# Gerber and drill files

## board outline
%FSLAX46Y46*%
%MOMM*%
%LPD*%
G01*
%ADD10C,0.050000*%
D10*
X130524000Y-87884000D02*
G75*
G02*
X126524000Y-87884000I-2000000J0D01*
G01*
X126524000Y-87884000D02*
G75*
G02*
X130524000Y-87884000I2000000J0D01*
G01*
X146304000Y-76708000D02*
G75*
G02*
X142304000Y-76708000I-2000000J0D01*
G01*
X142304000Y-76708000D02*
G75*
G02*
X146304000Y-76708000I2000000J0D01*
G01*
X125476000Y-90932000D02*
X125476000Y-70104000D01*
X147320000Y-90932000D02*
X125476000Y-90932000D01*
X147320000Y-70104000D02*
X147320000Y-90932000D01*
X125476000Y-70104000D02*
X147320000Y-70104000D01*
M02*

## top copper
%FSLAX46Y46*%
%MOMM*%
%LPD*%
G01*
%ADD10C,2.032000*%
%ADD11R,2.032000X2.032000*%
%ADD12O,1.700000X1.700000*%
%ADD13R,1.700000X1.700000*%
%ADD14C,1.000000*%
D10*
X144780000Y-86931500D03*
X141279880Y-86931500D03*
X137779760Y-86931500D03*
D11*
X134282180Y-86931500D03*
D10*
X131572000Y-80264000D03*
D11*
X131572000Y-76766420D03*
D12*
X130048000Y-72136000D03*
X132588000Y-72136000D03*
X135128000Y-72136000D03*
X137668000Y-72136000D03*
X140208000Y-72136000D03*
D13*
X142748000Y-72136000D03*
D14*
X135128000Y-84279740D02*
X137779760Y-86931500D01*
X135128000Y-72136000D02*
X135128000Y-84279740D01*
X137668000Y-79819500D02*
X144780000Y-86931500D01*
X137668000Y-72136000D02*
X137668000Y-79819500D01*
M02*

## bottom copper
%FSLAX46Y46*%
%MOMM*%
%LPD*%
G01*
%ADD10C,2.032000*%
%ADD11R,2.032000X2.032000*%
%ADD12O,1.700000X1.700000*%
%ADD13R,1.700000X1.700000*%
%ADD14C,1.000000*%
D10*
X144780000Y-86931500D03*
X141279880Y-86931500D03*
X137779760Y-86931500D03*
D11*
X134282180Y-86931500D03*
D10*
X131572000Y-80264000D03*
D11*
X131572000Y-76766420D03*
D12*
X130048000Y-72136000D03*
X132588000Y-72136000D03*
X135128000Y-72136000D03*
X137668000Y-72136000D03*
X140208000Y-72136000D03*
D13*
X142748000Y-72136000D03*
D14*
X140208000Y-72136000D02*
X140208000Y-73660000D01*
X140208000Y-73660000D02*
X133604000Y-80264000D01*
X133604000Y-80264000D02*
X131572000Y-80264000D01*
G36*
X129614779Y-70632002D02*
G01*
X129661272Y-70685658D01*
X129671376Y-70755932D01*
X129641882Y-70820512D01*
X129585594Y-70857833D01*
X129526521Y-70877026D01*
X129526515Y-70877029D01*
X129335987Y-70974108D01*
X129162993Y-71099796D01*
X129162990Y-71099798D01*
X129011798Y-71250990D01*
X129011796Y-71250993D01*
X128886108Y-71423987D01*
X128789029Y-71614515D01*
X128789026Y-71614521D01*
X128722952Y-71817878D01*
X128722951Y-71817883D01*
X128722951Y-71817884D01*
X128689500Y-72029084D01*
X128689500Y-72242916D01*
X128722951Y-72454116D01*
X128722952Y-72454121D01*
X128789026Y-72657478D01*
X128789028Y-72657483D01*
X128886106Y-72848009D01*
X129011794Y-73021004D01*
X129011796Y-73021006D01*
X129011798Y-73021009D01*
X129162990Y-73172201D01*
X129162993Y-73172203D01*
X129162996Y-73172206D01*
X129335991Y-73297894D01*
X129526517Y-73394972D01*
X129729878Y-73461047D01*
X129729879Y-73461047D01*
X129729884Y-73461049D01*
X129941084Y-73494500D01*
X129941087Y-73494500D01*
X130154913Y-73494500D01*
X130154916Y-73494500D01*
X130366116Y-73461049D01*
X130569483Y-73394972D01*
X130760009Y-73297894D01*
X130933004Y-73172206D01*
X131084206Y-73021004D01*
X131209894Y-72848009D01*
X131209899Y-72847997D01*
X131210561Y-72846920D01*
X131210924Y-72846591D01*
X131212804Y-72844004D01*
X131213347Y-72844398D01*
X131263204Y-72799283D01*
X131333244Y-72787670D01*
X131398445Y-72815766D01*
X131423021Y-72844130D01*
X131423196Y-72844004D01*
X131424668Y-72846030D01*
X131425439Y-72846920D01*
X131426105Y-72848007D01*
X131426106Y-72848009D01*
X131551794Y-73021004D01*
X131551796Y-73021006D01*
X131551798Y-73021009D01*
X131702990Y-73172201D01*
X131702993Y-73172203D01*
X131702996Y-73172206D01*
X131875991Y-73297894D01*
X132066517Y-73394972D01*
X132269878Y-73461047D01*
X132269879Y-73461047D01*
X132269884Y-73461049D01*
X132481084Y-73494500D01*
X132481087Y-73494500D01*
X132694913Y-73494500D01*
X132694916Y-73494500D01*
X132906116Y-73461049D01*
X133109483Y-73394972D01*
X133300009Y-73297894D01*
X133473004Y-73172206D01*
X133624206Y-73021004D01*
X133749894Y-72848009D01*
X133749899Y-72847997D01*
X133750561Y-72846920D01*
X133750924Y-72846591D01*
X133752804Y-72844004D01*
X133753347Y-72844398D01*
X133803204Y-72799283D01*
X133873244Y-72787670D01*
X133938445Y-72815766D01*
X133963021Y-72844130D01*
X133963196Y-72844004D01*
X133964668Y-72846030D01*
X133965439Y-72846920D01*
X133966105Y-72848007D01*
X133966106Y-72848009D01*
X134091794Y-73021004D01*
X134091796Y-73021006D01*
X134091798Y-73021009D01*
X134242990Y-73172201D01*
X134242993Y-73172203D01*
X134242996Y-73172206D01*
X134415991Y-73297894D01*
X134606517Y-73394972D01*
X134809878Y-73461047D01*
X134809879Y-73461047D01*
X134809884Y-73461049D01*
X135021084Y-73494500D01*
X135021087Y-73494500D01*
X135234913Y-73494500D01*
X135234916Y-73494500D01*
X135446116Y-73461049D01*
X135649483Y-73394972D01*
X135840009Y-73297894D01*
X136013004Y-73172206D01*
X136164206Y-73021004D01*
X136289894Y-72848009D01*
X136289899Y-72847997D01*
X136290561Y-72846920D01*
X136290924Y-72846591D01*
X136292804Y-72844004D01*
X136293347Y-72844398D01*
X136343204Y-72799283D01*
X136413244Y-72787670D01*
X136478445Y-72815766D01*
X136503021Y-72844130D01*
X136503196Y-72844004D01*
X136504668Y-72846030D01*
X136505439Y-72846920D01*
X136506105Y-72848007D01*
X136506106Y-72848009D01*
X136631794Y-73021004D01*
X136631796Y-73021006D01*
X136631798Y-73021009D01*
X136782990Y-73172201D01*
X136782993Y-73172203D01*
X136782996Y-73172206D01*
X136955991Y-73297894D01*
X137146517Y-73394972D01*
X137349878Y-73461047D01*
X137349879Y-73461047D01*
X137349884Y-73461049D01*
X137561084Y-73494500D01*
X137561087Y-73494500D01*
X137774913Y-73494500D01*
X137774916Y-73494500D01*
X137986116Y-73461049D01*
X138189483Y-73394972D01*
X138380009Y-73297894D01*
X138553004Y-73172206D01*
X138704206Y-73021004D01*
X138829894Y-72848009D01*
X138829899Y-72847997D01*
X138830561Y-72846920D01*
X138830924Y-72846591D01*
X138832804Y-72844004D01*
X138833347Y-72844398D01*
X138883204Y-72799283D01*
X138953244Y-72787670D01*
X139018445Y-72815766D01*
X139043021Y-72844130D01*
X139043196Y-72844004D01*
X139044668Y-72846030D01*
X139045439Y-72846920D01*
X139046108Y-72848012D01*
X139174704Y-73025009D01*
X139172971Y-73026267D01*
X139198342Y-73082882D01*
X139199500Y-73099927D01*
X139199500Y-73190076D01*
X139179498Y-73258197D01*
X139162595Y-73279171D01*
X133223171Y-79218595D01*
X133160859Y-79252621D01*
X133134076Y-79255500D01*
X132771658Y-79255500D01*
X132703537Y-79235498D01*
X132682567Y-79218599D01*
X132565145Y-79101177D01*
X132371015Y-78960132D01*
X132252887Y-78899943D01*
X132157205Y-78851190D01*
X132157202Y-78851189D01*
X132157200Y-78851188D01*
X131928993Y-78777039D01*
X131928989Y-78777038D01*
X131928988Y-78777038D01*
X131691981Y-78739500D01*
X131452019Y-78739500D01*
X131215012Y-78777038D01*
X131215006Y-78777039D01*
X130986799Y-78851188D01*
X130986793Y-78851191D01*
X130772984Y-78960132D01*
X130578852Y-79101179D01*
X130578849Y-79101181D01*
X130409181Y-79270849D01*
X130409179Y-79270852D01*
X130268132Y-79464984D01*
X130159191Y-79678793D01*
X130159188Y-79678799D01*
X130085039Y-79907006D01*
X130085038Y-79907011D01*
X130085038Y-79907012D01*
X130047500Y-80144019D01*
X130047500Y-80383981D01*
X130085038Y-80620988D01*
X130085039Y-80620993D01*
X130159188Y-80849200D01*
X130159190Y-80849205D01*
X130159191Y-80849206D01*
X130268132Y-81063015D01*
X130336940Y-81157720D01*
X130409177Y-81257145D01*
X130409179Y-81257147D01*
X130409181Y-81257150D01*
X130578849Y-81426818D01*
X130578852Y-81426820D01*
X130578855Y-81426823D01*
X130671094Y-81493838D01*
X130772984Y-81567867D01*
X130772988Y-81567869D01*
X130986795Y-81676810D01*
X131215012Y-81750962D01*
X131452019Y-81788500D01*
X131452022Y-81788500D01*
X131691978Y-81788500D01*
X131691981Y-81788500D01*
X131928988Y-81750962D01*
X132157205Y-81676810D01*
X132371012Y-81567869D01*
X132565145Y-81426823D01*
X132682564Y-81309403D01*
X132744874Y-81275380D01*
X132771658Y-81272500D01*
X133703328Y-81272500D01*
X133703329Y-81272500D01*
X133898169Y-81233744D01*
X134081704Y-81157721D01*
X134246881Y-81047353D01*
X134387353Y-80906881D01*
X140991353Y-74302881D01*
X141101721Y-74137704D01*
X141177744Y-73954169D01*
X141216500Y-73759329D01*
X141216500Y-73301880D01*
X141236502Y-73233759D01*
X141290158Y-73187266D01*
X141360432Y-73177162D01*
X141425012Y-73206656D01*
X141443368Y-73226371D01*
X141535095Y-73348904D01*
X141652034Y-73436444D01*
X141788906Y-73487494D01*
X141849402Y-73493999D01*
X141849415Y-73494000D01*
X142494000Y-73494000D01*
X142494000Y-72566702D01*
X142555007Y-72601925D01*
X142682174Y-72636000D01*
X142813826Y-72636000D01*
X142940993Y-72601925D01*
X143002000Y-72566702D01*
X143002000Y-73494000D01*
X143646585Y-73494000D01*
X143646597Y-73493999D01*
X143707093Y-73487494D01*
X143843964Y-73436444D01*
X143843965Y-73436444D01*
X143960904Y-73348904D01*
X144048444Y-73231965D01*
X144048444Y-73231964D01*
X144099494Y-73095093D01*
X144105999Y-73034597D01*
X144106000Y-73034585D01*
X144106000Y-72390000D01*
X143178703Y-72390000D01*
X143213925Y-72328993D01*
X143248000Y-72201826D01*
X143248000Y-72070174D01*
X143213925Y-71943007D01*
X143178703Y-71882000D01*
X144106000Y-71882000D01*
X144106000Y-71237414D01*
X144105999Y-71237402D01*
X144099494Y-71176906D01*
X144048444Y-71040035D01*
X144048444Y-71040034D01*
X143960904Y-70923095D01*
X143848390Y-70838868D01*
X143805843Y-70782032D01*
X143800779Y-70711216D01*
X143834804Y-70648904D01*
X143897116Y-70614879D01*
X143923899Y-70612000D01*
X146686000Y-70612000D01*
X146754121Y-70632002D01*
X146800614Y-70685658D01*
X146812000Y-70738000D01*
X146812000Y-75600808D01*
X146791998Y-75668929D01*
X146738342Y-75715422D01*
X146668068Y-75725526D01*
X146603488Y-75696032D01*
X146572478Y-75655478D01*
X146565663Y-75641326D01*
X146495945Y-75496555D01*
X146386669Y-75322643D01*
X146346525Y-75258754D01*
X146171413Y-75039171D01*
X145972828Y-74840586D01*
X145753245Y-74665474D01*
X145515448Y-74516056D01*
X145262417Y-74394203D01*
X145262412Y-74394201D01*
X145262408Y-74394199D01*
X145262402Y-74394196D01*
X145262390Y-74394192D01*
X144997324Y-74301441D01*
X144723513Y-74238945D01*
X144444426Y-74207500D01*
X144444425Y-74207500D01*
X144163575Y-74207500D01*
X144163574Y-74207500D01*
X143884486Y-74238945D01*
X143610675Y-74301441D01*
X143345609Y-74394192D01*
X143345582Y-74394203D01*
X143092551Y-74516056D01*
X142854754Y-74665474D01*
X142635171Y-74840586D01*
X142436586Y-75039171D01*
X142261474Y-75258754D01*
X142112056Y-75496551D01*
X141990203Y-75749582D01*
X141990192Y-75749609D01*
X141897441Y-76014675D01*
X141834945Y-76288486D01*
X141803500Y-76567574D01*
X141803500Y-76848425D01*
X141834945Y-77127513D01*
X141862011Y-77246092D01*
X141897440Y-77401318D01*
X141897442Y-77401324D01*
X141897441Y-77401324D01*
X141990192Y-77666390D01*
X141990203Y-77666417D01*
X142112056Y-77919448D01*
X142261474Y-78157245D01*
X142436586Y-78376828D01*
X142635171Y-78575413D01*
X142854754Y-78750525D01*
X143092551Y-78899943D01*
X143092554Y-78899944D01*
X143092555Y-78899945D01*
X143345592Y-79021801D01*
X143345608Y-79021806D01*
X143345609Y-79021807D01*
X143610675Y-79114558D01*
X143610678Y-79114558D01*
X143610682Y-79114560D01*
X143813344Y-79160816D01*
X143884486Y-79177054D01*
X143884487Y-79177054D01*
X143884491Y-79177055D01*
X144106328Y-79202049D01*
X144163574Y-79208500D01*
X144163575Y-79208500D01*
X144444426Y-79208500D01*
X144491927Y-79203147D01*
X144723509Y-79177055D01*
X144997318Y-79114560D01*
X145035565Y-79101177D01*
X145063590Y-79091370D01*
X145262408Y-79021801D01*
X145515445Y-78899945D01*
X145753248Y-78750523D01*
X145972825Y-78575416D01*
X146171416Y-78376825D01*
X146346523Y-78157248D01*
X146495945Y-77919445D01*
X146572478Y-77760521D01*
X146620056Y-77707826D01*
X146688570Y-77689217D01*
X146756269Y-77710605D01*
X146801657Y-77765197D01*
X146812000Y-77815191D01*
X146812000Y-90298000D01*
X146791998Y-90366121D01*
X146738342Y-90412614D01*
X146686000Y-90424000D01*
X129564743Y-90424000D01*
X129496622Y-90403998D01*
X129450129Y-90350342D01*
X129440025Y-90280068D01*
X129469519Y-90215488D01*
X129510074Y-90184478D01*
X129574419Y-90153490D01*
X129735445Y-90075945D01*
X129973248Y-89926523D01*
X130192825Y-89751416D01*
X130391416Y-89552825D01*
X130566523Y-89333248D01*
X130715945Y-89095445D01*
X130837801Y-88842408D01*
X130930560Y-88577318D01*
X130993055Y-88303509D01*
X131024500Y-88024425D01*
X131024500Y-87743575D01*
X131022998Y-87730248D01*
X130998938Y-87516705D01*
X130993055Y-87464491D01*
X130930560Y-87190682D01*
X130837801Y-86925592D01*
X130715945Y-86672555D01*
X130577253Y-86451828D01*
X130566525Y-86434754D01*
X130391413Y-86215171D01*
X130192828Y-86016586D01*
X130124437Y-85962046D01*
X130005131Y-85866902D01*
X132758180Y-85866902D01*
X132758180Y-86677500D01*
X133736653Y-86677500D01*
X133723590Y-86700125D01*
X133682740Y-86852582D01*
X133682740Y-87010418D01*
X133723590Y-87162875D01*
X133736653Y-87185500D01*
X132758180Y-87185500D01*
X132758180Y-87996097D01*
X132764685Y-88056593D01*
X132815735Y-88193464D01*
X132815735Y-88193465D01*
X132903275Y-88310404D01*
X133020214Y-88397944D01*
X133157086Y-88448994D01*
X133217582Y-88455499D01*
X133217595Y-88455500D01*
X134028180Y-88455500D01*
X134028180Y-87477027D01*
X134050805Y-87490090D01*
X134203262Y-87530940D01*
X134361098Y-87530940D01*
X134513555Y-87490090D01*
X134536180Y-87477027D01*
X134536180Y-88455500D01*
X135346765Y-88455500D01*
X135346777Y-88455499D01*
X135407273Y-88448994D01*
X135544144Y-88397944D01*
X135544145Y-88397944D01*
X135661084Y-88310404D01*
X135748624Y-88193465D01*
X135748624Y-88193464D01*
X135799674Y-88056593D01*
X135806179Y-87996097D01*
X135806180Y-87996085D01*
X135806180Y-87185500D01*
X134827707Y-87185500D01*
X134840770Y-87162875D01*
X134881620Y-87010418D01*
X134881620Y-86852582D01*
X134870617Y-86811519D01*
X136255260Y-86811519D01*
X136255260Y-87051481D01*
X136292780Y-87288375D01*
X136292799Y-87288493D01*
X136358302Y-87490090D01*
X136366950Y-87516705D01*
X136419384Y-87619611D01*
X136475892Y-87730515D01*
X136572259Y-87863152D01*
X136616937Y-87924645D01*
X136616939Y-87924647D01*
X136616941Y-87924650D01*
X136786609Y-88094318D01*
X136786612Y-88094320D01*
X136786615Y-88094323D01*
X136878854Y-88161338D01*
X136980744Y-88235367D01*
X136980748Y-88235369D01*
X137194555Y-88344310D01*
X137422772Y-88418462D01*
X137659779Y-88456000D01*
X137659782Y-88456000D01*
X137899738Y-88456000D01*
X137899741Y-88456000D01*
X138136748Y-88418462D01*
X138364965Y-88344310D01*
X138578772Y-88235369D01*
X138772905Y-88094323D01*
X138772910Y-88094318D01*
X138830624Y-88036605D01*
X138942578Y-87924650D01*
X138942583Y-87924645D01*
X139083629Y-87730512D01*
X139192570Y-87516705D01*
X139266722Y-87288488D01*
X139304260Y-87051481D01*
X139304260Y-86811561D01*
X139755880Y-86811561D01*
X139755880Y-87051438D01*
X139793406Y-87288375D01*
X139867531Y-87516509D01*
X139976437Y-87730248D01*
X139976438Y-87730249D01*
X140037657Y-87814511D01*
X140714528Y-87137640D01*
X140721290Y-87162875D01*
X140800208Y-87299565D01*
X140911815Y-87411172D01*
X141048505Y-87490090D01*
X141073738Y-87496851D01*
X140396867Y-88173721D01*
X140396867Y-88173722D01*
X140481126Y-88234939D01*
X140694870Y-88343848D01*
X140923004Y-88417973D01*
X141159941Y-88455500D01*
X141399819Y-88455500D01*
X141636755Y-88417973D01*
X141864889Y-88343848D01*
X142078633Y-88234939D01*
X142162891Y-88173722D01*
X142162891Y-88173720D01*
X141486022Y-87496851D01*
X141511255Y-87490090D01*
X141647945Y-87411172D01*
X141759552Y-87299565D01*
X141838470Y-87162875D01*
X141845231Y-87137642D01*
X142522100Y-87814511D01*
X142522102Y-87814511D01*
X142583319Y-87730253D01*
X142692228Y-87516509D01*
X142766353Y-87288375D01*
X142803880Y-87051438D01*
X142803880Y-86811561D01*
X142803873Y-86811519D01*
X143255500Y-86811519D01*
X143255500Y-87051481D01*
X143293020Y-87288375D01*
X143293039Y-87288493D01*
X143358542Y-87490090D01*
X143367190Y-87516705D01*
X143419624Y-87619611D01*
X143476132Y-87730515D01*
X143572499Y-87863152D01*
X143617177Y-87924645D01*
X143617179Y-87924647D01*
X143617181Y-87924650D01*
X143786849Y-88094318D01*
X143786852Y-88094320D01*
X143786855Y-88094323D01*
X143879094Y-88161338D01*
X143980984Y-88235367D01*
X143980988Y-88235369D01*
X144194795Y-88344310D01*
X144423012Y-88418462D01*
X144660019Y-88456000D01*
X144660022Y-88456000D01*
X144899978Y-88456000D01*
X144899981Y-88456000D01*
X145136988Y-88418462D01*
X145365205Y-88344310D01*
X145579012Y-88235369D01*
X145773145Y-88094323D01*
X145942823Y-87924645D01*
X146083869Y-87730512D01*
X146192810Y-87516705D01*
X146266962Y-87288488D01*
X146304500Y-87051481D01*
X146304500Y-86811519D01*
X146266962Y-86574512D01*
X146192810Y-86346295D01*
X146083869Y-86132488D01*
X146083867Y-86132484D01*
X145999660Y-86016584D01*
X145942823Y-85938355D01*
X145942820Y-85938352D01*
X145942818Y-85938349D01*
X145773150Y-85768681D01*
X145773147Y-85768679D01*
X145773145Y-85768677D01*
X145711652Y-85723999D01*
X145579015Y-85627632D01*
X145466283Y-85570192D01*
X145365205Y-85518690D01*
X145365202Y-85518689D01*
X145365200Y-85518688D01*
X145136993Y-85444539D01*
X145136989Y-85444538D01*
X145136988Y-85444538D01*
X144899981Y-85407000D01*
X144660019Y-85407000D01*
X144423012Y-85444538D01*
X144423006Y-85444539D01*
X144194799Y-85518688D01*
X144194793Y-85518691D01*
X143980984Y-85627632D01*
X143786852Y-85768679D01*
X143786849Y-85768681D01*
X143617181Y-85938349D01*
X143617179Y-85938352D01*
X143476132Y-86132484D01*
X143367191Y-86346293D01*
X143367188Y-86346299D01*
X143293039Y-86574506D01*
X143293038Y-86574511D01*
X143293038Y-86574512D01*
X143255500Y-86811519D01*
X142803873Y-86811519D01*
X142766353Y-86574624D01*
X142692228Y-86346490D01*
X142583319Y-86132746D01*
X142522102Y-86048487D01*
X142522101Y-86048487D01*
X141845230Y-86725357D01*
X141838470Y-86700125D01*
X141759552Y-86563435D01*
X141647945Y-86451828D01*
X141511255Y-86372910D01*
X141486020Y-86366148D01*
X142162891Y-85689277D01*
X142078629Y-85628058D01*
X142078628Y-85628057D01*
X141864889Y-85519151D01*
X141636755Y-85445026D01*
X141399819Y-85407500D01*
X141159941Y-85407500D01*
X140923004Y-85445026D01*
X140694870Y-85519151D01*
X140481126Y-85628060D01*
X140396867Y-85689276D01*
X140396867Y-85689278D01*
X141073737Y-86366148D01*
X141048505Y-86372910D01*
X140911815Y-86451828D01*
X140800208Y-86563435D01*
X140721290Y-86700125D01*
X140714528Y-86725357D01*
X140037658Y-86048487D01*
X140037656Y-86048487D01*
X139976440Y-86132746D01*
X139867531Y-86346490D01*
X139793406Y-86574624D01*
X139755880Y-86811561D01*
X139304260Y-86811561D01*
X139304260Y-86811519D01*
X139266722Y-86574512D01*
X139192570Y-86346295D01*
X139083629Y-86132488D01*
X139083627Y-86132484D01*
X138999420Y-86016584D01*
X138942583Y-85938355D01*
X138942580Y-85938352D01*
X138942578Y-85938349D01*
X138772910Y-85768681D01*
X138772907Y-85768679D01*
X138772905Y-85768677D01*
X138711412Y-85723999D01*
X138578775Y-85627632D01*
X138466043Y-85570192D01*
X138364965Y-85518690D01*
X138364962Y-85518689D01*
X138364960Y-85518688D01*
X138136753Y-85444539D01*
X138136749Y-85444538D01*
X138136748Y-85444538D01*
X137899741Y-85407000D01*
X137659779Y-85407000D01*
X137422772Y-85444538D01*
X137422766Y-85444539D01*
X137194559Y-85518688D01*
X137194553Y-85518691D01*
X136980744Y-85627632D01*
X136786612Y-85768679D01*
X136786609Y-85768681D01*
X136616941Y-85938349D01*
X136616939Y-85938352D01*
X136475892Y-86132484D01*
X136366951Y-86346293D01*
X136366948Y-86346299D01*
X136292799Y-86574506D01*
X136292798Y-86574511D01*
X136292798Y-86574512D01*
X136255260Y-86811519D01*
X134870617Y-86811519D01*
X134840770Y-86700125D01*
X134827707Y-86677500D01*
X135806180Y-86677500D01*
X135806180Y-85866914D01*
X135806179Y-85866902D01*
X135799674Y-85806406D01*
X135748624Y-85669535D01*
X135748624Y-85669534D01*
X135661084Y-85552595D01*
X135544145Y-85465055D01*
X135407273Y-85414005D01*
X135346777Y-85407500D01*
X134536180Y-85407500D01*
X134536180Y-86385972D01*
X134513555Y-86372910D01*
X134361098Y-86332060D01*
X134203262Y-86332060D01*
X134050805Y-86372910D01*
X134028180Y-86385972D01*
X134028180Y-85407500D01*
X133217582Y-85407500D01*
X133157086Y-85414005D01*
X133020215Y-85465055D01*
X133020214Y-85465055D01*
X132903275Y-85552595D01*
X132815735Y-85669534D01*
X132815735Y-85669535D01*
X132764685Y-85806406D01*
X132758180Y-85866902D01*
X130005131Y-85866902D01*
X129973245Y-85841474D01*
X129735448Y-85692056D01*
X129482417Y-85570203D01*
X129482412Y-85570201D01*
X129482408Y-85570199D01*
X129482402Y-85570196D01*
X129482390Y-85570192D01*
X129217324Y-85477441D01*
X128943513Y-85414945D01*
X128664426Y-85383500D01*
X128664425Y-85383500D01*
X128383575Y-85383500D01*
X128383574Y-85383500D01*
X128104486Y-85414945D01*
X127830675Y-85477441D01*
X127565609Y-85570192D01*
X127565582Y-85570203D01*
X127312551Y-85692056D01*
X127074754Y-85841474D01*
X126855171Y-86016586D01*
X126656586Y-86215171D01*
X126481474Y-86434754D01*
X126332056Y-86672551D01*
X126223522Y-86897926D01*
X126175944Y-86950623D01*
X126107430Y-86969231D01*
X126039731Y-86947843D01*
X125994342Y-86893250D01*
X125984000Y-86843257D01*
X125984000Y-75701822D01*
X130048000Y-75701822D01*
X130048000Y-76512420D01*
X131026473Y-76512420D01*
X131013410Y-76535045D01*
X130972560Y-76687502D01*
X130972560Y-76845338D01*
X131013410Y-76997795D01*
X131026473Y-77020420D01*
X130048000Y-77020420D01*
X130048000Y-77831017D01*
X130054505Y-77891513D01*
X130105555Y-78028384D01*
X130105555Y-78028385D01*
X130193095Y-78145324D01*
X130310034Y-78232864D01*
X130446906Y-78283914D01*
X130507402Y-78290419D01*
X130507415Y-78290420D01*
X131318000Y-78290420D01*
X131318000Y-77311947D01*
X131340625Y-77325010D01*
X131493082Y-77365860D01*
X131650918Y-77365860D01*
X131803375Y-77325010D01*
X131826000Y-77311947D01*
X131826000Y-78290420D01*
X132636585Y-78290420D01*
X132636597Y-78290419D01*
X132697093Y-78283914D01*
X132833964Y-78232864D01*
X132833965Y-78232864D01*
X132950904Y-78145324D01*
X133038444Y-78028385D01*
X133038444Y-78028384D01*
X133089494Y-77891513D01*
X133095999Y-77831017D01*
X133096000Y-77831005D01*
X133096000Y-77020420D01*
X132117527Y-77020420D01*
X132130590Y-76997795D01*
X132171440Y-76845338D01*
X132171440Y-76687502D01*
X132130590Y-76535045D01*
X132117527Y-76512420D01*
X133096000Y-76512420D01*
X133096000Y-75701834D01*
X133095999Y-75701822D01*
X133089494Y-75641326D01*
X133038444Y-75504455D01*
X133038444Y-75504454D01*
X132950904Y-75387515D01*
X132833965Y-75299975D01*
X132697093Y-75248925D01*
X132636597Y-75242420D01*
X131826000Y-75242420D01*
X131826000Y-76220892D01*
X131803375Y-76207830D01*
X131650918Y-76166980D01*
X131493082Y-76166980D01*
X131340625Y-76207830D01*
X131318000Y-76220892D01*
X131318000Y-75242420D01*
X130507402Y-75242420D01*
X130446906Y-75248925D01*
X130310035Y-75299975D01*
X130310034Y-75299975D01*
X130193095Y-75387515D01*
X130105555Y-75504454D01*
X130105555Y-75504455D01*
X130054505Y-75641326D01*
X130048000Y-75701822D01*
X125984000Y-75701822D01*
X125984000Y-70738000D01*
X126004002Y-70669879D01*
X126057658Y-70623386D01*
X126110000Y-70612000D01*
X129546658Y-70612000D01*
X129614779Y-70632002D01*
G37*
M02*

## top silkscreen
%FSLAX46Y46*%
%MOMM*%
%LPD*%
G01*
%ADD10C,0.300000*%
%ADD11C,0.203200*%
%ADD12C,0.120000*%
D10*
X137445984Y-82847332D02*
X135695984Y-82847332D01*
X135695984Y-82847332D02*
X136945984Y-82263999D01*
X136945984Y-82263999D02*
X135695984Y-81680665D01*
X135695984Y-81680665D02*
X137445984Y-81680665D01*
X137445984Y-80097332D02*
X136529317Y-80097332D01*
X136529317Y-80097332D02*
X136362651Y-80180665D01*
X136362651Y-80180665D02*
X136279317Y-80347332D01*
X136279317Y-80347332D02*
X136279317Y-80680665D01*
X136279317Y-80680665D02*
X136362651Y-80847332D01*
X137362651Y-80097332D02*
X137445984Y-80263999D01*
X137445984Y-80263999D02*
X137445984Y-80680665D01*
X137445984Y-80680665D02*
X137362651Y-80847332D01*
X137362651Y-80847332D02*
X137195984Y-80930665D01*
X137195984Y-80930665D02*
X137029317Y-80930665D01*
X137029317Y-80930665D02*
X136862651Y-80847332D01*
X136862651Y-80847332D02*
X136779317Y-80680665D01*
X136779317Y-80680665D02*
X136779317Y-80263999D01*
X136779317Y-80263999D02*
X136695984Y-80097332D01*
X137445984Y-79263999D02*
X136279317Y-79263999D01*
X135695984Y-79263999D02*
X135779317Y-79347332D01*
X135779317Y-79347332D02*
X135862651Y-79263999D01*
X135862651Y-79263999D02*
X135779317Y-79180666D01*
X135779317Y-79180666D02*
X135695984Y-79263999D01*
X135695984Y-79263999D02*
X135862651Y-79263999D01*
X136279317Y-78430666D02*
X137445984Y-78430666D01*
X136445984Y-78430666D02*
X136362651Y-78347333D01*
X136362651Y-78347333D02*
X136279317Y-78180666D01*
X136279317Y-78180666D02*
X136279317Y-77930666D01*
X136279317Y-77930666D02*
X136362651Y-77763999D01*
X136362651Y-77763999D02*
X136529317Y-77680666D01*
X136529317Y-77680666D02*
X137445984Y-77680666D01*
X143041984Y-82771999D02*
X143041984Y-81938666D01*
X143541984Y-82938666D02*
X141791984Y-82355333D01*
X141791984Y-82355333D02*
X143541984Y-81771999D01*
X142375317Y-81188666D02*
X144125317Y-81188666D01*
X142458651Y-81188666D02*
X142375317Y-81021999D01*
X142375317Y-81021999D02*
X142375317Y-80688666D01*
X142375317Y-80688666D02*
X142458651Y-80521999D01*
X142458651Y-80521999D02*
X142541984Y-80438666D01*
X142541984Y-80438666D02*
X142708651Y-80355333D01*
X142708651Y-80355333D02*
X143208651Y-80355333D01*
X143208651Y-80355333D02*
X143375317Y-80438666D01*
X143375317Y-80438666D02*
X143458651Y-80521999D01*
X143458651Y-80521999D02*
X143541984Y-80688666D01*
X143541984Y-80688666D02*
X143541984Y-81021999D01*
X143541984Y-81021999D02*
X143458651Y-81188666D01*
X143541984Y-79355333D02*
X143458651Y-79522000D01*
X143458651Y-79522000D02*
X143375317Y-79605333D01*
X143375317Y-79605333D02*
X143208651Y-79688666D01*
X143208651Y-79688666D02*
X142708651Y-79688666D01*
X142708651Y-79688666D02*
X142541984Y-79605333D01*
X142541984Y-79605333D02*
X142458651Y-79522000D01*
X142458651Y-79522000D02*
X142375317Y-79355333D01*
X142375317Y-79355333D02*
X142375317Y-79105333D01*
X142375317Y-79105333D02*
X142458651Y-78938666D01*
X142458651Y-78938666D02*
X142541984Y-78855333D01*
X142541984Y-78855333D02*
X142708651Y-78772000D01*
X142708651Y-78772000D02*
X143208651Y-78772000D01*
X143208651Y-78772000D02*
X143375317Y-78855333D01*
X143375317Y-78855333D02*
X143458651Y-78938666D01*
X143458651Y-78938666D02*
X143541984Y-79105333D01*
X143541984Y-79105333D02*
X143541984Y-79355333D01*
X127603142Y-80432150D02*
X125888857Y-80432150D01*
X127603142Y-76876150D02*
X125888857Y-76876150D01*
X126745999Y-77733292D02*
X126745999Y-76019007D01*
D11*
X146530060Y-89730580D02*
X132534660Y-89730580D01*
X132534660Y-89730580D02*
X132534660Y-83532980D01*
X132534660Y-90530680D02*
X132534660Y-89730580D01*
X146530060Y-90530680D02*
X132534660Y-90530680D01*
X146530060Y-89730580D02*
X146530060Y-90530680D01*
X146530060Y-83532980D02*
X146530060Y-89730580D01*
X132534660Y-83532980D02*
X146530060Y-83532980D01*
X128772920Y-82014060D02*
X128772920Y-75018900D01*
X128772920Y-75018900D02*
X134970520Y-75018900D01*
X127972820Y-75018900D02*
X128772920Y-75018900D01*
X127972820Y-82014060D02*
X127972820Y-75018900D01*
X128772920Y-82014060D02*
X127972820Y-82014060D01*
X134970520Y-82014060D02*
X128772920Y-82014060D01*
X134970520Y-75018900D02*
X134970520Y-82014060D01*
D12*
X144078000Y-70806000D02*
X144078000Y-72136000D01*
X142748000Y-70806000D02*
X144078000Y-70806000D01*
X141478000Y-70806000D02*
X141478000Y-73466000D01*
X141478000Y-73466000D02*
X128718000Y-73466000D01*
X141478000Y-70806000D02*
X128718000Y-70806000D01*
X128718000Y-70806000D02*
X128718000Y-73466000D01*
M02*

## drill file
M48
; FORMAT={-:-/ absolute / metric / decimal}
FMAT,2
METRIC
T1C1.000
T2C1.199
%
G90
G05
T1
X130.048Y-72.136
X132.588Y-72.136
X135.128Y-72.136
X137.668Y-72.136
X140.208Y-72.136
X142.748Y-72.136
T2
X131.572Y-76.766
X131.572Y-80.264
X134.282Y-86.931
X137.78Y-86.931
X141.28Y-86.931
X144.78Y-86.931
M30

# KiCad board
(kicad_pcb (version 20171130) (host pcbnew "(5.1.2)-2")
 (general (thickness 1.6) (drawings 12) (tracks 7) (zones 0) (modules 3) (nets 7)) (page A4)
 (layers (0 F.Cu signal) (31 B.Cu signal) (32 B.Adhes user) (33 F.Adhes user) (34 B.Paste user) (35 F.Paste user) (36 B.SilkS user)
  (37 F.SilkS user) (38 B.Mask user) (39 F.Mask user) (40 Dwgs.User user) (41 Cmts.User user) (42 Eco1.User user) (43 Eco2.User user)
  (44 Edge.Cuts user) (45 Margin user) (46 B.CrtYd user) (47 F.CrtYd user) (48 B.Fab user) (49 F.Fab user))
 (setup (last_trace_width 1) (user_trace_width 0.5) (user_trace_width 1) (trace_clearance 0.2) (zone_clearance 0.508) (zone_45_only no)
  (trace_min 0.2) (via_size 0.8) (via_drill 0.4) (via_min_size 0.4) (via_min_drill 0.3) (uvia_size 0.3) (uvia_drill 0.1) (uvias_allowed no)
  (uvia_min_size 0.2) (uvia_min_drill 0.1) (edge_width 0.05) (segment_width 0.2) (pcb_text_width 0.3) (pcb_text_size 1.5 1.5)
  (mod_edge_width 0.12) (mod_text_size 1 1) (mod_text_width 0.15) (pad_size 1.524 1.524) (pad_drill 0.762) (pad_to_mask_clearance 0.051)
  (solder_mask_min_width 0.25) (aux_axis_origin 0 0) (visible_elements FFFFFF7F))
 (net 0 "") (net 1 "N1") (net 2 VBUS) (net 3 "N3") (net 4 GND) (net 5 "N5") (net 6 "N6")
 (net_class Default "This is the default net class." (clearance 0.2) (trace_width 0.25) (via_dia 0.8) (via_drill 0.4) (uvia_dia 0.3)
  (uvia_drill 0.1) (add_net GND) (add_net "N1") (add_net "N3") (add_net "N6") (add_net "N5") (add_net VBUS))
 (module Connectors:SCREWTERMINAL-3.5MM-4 (layer F.Cu) (at 134.28218 86.9315)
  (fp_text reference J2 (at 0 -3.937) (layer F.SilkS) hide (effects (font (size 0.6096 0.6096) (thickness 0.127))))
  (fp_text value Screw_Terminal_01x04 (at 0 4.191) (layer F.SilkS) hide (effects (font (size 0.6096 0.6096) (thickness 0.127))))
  (fp_line (start 12.24788 2.79908) (end -1.74752 2.79908) (layer F.SilkS) (width 0.2032))
  (fp_line (start -1.74752 2.79908) (end -1.74752 -3.39852) (layer F.SilkS) (width 0.2032))
  (fp_line (start -1.74752 3.59918) (end -1.74752 2.79908) (layer F.SilkS) (width 0.2032))
  (fp_line (start 12.24788 3.59918) (end -1.74752 3.59918) (layer F.SilkS) (width 0.2032))
  (fp_line (start 12.24788 2.79908) (end 12.24788 3.59918) (layer F.SilkS) (width 0.2032))
  (fp_line (start 12.24788 -3.39852) (end 12.24788 2.79908) (layer F.SilkS) (width 0.2032))
  (fp_line (start -1.74752 -3.39852) (end 12.24788 -3.39852) (layer F.SilkS) (width 0.2032))
  (pad 4 thru_hole circle (at 10.49782 0) (size 2.032 2.032) (drill 1.19888) (layers *.Cu *.Mask) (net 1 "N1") (solder_mask_margin 0.1016))
  (pad 3 thru_hole circle (at 6.9977 0) (size 2.032 2.032) (drill 1.19888) (layers *.Cu *.Mask) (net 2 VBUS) (solder_mask_margin 0.1016))
  (pad 2 thru_hole circle (at 3.49758 0) (size 2.032 2.032) (drill 1.19888) (layers *.Cu *.Mask) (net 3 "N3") (solder_mask_margin 0.1016))
  (pad 1 thru_hole rect (at 0 0) (size 2.032 2.032) (drill 1.19888) (layers *.Cu *.Mask) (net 2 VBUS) (solder_mask_margin 0.1016)))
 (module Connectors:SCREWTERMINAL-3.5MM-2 (layer F.Cu) (at 131.572 76.76642 270)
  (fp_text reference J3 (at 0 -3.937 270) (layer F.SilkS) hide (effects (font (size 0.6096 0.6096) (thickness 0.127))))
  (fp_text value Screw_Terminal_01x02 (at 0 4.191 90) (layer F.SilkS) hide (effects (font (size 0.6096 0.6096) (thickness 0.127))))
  (fp_line (start 5.24764 2.79908) (end -1.74752 2.79908) (layer F.SilkS) (width 0.2032))
  (fp_line (start -1.74752 2.79908) (end -1.74752 -3.39852) (layer F.SilkS) (width 0.2032))
  (fp_line (start -1.74752 3.59918) (end -1.74752 2.79908) (layer F.SilkS) (width 0.2032))
  (fp_line (start 5.24764 3.59918) (end -1.74752 3.59918) (layer F.SilkS) (width 0.2032))
  (fp_line (start 5.24764 2.79908) (end 5.24764 3.59918) (layer F.SilkS) (width 0.2032))
  (fp_line (start 5.24764 -3.39852) (end 5.24764 2.79908) (layer F.SilkS) (width 0.2032))
  (fp_line (start -1.74752 -3.39852) (end 5.24764 -3.39852) (layer F.SilkS) (width 0.2032))
  (pad 2 thru_hole circle (at 3.49758 0 270) (size 2.032 2.032) (drill 1.19888) (layers *.Cu *.Mask) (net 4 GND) (solder_mask_margin 0.1016))
  (pad 1 thru_hole rect (at 0 0 270) (size 2.032 2.032) (drill 1.19888) (layers *.Cu *.Mask) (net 2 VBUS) (solder_mask_margin 0.1016)))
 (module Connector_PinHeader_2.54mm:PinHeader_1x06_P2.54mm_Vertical (layer F.Cu) (at 142.748 72.136 270)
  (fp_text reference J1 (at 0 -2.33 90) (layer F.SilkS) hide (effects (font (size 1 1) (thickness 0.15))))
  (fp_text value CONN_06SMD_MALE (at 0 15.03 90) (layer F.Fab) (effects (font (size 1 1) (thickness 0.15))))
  (fp_line (start -1.33 -1.33) (end 0 -1.33) (layer F.SilkS) (width 0.12))
  (fp_line (start -1.33 0) (end -1.33 -1.33) (layer F.SilkS) (width 0.12))
  (fp_line (start -1.33 1.27) (end 1.33 1.27) (layer F.SilkS) (width 0.12))
  (fp_line (start 1.33 1.27) (end 1.33 14.03) (layer F.SilkS) (width 0.12))
  (fp_line (start -1.33 1.27) (end -1.33 14.03) (layer F.SilkS) (width 0.12))
  (fp_line (start -1.33 14.03) (end 1.33 14.03) (layer F.SilkS) (width 0.12))
  (pad 6 thru_hole oval (at 0 12.7 270) (size 1.7 1.7) (drill 1) (layers *.Cu *.Mask) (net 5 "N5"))
  (pad 5 thru_hole oval (at 0 10.16 270) (size 1.7 1.7) (drill 1) (layers *.Cu *.Mask) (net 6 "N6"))
  (pad 4 thru_hole oval (at 0 7.62 270) (size 1.7 1.7) (drill 1) (layers *.Cu *.Mask) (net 3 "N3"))
  (pad 3 thru_hole oval (at 0 5.08 270) (size 1.7 1.7) (drill 1) (layers *.Cu *.Mask) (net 1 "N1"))
  (pad 2 thru_hole oval (at 0 2.54 270) (size 1.7 1.7) (drill 1) (layers *.Cu *.Mask) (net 4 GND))
  (pad 1 thru_hole rect (at 0 0 270) (size 1.7 1.7) (drill 1) (layers *.Cu *.Mask) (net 2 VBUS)))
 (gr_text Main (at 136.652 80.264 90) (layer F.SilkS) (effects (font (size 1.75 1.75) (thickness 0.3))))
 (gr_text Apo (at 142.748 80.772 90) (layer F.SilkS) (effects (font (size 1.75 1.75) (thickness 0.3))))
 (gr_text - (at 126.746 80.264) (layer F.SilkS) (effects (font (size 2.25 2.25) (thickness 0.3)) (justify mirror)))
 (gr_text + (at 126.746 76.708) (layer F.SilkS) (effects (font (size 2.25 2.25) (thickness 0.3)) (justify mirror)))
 (gr_circle (center 128.524 87.884) (end 130.524 87.884) (layer Edge.Cuts) (width 0.05))
 (gr_circle (center 144.304 76.708) (end 146.304 76.708) (layer Edge.Cuts) (width 0.05))
 (gr_line (start 125.476 90.932) (end 125.476 70.104) (layer Edge.Cuts) (width 0.05))
 (gr_line (start 147.32 90.932) (end 125.476 90.932) (layer Edge.Cuts) (width 0.05))
 (gr_line (start 147.32 70.104) (end 147.32 90.932) (layer Edge.Cuts) (width 0.05))
 (gr_line (start 125.476 70.104) (end 147.32 70.104) (layer Edge.Cuts) (width 0.05))
 (segment (start 135.128 84.27974) (end 137.77976 86.9315) (width 1) (layer F.Cu) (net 3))
 (segment (start 135.128 72.136) (end 135.128 84.27974) (width 1) (layer F.Cu) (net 3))
 (segment (start 137.668 79.8195) (end 144.78 86.9315) (width 1) (layer F.Cu) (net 1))
 (segment (start 137.668 72.136) (end 137.668 79.8195) (width 1) (layer F.Cu) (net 1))
 (segment (start 140.208 72.136) (end 140.208 73.66) (width 1) (layer B.Cu) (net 4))
 (segment (start 140.208 73.66) (end 133.604 80.264) (width 1) (layer B.Cu) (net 4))
 (segment (start 133.604 80.264) (end 131.572 80.264) (width 1) (layer B.Cu) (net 4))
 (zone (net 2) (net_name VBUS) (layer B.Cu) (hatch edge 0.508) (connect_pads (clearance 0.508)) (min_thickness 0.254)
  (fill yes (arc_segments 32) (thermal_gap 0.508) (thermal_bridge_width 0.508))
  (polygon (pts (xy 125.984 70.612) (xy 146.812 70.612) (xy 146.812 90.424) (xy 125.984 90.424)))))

